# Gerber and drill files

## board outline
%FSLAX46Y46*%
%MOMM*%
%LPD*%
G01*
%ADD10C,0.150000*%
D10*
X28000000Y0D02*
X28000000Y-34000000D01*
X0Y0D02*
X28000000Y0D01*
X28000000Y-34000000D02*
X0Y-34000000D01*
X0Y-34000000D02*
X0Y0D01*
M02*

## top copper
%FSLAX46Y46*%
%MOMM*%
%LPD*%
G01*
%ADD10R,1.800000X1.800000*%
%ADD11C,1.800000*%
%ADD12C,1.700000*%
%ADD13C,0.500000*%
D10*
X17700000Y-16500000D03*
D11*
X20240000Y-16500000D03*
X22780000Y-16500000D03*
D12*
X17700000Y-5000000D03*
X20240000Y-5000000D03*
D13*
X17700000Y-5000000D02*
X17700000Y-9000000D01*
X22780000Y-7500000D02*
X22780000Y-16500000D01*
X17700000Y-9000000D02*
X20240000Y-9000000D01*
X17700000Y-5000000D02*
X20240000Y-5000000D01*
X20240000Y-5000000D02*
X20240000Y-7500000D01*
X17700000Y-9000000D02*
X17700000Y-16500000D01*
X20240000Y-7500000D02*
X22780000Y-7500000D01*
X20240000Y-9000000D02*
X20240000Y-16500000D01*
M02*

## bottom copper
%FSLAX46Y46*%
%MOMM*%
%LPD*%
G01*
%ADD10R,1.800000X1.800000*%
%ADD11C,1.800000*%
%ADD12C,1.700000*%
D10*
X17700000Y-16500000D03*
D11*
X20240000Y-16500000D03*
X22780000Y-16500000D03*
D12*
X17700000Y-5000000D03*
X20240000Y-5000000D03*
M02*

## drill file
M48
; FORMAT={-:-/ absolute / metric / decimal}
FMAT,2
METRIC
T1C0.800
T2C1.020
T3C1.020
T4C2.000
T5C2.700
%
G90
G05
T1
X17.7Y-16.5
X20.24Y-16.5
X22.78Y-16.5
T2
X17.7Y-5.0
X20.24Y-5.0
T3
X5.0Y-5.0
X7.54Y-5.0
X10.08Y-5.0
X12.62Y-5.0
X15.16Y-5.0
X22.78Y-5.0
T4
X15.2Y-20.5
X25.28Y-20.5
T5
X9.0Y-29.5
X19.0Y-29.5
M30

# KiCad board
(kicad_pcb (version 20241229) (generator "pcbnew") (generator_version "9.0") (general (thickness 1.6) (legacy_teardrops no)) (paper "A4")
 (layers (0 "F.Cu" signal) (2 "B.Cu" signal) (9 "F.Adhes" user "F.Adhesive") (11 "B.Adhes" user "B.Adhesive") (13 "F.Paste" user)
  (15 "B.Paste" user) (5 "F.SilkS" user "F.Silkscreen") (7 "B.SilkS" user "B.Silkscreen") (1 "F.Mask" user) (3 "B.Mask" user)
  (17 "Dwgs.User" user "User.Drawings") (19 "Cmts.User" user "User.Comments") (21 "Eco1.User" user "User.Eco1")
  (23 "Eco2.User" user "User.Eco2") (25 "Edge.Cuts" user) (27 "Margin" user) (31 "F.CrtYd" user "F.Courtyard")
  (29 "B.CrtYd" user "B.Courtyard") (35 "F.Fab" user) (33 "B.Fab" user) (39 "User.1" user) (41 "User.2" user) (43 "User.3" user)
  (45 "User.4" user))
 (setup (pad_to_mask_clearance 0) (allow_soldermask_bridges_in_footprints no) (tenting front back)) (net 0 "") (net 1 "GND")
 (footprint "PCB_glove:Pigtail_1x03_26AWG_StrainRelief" (layer "F.Cu") (at 17.7 16.5)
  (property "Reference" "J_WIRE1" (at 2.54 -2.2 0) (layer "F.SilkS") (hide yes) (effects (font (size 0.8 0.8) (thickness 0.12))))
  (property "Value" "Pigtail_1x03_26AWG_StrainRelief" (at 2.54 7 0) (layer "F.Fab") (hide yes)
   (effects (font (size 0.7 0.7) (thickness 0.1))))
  (pad "" np_thru_hole circle (at -2.5 4) (size 2 2) (drill 2) (layers "*.Cu" "*.Mask"))
  (pad "" np_thru_hole circle (at 7.58 4) (size 2 2) (drill 2) (layers "*.Cu" "*.Mask"))
  (pad "1" thru_hole rect (at 0 0) (size 1.8 1.8) (drill 0.8) (layers "*.Cu" "*.Mask") (remove_unused_layers no) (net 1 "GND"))
  (pad "2" thru_hole circle (at 2.54 0) (size 1.8 1.8) (drill 0.8) (layers "*.Cu" "*.Mask") (remove_unused_layers no) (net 1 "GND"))
  (pad "3" thru_hole circle (at 5.08 0) (size 1.8 1.8) (drill 0.8) (layers "*.Cu" "*.Mask") (remove_unused_layers no) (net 1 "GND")))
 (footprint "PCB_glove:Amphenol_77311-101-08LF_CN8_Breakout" (layer "F.Cu") (at 5 5)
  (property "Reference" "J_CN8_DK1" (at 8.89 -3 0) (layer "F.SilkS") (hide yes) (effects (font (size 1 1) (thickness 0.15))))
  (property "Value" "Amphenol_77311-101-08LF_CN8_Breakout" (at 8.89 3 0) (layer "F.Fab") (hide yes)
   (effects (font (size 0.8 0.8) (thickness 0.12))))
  (pad "" np_thru_hole circle (at 0 0) (size 1.02 1.02) (drill 1.02) (layers "*.Cu" "*.Mask"))
  (pad "" np_thru_hole circle (at 2.54 0) (size 1.02 1.02) (drill 1.02) (layers "*.Cu" "*.Mask"))
  (pad "" np_thru_hole circle (at 5.08 0) (size 1.02 1.02) (drill 1.02) (layers "*.Cu" "*.Mask"))
  (pad "" np_thru_hole circle (at 7.62 0) (size 1.02 1.02) (drill 1.02) (layers "*.Cu" "*.Mask"))
  (pad "" np_thru_hole circle (at 10.16 0) (size 1.02 1.02) (drill 1.02) (layers "*.Cu" "*.Mask"))
  (pad "" np_thru_hole circle (at 17.78 0) (size 1.02 1.02) (drill 1.02) (layers "*.Cu" "*.Mask"))
  (pad "6" thru_hole circle (at 12.7 0) (size 1.7 1.7) (drill 1.02) (layers "*.Cu" "*.Mask") (remove_unused_layers no) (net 1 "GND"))
  (pad "7" thru_hole circle (at 15.24 0) (size 1.7 1.7) (drill 1.02) (layers "*.Cu" "*.Mask") (remove_unused_layers no) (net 1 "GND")))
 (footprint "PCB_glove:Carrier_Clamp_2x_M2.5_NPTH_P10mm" (layer "F.Cu") (at 14 29.5)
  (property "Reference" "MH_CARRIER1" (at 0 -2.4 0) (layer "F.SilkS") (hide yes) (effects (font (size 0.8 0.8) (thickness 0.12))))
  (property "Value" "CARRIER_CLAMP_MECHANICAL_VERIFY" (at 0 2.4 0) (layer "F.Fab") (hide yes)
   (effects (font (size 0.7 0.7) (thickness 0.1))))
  (pad "" np_thru_hole circle (at -5 0) (size 2.7 2.7) (drill 2.7) (layers "*.Cu" "*.Mask"))
  (pad "" np_thru_hole circle (at 5 0) (size 2.7 2.7) (drill 2.7) (layers "*.Cu" "*.Mask")))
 (gr_line (start 28 0) (end 28 34) (stroke (width 0.15) (type default)) (layer "Edge.Cuts"))
 (gr_line (start 0 0) (end 28 0) (stroke (width 0.15) (type default)) (layer "Edge.Cuts"))
 (gr_line (start 28 34) (end 0 34) (stroke (width 0.15) (type default)) (layer "Edge.Cuts"))
 (gr_line (start 0 34) (end 0 0) (stroke (width 0.15) (type default)) (layer "Edge.Cuts"))
 (segment (start 17.7 5) (end 17.7 9) (width 0.5) (layer "F.Cu") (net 1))
 (segment (start 22.78 7.5) (end 22.78 16.5) (width 0.5) (layer "F.Cu") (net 1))
 (segment (start 17.7 9) (end 20.24 9) (width 0.5) (layer "F.Cu") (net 1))
 (segment (start 17.7 5) (end 20.24 5) (width 0.5) (layer "F.Cu") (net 1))
 (segment (start 20.24 5) (end 20.24 7.5) (width 0.5) (layer "F.Cu") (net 1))
 (segment (start 17.7 9) (end 17.7 16.5) (width 0.5) (layer "F.Cu") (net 1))
 (segment (start 20.24 7.5) (end 22.78 7.5) (width 0.5) (layer "F.Cu") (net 1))
 (segment (start 20.24 9) (end 20.24 16.5) (width 0.5) (layer "F.Cu") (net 1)))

